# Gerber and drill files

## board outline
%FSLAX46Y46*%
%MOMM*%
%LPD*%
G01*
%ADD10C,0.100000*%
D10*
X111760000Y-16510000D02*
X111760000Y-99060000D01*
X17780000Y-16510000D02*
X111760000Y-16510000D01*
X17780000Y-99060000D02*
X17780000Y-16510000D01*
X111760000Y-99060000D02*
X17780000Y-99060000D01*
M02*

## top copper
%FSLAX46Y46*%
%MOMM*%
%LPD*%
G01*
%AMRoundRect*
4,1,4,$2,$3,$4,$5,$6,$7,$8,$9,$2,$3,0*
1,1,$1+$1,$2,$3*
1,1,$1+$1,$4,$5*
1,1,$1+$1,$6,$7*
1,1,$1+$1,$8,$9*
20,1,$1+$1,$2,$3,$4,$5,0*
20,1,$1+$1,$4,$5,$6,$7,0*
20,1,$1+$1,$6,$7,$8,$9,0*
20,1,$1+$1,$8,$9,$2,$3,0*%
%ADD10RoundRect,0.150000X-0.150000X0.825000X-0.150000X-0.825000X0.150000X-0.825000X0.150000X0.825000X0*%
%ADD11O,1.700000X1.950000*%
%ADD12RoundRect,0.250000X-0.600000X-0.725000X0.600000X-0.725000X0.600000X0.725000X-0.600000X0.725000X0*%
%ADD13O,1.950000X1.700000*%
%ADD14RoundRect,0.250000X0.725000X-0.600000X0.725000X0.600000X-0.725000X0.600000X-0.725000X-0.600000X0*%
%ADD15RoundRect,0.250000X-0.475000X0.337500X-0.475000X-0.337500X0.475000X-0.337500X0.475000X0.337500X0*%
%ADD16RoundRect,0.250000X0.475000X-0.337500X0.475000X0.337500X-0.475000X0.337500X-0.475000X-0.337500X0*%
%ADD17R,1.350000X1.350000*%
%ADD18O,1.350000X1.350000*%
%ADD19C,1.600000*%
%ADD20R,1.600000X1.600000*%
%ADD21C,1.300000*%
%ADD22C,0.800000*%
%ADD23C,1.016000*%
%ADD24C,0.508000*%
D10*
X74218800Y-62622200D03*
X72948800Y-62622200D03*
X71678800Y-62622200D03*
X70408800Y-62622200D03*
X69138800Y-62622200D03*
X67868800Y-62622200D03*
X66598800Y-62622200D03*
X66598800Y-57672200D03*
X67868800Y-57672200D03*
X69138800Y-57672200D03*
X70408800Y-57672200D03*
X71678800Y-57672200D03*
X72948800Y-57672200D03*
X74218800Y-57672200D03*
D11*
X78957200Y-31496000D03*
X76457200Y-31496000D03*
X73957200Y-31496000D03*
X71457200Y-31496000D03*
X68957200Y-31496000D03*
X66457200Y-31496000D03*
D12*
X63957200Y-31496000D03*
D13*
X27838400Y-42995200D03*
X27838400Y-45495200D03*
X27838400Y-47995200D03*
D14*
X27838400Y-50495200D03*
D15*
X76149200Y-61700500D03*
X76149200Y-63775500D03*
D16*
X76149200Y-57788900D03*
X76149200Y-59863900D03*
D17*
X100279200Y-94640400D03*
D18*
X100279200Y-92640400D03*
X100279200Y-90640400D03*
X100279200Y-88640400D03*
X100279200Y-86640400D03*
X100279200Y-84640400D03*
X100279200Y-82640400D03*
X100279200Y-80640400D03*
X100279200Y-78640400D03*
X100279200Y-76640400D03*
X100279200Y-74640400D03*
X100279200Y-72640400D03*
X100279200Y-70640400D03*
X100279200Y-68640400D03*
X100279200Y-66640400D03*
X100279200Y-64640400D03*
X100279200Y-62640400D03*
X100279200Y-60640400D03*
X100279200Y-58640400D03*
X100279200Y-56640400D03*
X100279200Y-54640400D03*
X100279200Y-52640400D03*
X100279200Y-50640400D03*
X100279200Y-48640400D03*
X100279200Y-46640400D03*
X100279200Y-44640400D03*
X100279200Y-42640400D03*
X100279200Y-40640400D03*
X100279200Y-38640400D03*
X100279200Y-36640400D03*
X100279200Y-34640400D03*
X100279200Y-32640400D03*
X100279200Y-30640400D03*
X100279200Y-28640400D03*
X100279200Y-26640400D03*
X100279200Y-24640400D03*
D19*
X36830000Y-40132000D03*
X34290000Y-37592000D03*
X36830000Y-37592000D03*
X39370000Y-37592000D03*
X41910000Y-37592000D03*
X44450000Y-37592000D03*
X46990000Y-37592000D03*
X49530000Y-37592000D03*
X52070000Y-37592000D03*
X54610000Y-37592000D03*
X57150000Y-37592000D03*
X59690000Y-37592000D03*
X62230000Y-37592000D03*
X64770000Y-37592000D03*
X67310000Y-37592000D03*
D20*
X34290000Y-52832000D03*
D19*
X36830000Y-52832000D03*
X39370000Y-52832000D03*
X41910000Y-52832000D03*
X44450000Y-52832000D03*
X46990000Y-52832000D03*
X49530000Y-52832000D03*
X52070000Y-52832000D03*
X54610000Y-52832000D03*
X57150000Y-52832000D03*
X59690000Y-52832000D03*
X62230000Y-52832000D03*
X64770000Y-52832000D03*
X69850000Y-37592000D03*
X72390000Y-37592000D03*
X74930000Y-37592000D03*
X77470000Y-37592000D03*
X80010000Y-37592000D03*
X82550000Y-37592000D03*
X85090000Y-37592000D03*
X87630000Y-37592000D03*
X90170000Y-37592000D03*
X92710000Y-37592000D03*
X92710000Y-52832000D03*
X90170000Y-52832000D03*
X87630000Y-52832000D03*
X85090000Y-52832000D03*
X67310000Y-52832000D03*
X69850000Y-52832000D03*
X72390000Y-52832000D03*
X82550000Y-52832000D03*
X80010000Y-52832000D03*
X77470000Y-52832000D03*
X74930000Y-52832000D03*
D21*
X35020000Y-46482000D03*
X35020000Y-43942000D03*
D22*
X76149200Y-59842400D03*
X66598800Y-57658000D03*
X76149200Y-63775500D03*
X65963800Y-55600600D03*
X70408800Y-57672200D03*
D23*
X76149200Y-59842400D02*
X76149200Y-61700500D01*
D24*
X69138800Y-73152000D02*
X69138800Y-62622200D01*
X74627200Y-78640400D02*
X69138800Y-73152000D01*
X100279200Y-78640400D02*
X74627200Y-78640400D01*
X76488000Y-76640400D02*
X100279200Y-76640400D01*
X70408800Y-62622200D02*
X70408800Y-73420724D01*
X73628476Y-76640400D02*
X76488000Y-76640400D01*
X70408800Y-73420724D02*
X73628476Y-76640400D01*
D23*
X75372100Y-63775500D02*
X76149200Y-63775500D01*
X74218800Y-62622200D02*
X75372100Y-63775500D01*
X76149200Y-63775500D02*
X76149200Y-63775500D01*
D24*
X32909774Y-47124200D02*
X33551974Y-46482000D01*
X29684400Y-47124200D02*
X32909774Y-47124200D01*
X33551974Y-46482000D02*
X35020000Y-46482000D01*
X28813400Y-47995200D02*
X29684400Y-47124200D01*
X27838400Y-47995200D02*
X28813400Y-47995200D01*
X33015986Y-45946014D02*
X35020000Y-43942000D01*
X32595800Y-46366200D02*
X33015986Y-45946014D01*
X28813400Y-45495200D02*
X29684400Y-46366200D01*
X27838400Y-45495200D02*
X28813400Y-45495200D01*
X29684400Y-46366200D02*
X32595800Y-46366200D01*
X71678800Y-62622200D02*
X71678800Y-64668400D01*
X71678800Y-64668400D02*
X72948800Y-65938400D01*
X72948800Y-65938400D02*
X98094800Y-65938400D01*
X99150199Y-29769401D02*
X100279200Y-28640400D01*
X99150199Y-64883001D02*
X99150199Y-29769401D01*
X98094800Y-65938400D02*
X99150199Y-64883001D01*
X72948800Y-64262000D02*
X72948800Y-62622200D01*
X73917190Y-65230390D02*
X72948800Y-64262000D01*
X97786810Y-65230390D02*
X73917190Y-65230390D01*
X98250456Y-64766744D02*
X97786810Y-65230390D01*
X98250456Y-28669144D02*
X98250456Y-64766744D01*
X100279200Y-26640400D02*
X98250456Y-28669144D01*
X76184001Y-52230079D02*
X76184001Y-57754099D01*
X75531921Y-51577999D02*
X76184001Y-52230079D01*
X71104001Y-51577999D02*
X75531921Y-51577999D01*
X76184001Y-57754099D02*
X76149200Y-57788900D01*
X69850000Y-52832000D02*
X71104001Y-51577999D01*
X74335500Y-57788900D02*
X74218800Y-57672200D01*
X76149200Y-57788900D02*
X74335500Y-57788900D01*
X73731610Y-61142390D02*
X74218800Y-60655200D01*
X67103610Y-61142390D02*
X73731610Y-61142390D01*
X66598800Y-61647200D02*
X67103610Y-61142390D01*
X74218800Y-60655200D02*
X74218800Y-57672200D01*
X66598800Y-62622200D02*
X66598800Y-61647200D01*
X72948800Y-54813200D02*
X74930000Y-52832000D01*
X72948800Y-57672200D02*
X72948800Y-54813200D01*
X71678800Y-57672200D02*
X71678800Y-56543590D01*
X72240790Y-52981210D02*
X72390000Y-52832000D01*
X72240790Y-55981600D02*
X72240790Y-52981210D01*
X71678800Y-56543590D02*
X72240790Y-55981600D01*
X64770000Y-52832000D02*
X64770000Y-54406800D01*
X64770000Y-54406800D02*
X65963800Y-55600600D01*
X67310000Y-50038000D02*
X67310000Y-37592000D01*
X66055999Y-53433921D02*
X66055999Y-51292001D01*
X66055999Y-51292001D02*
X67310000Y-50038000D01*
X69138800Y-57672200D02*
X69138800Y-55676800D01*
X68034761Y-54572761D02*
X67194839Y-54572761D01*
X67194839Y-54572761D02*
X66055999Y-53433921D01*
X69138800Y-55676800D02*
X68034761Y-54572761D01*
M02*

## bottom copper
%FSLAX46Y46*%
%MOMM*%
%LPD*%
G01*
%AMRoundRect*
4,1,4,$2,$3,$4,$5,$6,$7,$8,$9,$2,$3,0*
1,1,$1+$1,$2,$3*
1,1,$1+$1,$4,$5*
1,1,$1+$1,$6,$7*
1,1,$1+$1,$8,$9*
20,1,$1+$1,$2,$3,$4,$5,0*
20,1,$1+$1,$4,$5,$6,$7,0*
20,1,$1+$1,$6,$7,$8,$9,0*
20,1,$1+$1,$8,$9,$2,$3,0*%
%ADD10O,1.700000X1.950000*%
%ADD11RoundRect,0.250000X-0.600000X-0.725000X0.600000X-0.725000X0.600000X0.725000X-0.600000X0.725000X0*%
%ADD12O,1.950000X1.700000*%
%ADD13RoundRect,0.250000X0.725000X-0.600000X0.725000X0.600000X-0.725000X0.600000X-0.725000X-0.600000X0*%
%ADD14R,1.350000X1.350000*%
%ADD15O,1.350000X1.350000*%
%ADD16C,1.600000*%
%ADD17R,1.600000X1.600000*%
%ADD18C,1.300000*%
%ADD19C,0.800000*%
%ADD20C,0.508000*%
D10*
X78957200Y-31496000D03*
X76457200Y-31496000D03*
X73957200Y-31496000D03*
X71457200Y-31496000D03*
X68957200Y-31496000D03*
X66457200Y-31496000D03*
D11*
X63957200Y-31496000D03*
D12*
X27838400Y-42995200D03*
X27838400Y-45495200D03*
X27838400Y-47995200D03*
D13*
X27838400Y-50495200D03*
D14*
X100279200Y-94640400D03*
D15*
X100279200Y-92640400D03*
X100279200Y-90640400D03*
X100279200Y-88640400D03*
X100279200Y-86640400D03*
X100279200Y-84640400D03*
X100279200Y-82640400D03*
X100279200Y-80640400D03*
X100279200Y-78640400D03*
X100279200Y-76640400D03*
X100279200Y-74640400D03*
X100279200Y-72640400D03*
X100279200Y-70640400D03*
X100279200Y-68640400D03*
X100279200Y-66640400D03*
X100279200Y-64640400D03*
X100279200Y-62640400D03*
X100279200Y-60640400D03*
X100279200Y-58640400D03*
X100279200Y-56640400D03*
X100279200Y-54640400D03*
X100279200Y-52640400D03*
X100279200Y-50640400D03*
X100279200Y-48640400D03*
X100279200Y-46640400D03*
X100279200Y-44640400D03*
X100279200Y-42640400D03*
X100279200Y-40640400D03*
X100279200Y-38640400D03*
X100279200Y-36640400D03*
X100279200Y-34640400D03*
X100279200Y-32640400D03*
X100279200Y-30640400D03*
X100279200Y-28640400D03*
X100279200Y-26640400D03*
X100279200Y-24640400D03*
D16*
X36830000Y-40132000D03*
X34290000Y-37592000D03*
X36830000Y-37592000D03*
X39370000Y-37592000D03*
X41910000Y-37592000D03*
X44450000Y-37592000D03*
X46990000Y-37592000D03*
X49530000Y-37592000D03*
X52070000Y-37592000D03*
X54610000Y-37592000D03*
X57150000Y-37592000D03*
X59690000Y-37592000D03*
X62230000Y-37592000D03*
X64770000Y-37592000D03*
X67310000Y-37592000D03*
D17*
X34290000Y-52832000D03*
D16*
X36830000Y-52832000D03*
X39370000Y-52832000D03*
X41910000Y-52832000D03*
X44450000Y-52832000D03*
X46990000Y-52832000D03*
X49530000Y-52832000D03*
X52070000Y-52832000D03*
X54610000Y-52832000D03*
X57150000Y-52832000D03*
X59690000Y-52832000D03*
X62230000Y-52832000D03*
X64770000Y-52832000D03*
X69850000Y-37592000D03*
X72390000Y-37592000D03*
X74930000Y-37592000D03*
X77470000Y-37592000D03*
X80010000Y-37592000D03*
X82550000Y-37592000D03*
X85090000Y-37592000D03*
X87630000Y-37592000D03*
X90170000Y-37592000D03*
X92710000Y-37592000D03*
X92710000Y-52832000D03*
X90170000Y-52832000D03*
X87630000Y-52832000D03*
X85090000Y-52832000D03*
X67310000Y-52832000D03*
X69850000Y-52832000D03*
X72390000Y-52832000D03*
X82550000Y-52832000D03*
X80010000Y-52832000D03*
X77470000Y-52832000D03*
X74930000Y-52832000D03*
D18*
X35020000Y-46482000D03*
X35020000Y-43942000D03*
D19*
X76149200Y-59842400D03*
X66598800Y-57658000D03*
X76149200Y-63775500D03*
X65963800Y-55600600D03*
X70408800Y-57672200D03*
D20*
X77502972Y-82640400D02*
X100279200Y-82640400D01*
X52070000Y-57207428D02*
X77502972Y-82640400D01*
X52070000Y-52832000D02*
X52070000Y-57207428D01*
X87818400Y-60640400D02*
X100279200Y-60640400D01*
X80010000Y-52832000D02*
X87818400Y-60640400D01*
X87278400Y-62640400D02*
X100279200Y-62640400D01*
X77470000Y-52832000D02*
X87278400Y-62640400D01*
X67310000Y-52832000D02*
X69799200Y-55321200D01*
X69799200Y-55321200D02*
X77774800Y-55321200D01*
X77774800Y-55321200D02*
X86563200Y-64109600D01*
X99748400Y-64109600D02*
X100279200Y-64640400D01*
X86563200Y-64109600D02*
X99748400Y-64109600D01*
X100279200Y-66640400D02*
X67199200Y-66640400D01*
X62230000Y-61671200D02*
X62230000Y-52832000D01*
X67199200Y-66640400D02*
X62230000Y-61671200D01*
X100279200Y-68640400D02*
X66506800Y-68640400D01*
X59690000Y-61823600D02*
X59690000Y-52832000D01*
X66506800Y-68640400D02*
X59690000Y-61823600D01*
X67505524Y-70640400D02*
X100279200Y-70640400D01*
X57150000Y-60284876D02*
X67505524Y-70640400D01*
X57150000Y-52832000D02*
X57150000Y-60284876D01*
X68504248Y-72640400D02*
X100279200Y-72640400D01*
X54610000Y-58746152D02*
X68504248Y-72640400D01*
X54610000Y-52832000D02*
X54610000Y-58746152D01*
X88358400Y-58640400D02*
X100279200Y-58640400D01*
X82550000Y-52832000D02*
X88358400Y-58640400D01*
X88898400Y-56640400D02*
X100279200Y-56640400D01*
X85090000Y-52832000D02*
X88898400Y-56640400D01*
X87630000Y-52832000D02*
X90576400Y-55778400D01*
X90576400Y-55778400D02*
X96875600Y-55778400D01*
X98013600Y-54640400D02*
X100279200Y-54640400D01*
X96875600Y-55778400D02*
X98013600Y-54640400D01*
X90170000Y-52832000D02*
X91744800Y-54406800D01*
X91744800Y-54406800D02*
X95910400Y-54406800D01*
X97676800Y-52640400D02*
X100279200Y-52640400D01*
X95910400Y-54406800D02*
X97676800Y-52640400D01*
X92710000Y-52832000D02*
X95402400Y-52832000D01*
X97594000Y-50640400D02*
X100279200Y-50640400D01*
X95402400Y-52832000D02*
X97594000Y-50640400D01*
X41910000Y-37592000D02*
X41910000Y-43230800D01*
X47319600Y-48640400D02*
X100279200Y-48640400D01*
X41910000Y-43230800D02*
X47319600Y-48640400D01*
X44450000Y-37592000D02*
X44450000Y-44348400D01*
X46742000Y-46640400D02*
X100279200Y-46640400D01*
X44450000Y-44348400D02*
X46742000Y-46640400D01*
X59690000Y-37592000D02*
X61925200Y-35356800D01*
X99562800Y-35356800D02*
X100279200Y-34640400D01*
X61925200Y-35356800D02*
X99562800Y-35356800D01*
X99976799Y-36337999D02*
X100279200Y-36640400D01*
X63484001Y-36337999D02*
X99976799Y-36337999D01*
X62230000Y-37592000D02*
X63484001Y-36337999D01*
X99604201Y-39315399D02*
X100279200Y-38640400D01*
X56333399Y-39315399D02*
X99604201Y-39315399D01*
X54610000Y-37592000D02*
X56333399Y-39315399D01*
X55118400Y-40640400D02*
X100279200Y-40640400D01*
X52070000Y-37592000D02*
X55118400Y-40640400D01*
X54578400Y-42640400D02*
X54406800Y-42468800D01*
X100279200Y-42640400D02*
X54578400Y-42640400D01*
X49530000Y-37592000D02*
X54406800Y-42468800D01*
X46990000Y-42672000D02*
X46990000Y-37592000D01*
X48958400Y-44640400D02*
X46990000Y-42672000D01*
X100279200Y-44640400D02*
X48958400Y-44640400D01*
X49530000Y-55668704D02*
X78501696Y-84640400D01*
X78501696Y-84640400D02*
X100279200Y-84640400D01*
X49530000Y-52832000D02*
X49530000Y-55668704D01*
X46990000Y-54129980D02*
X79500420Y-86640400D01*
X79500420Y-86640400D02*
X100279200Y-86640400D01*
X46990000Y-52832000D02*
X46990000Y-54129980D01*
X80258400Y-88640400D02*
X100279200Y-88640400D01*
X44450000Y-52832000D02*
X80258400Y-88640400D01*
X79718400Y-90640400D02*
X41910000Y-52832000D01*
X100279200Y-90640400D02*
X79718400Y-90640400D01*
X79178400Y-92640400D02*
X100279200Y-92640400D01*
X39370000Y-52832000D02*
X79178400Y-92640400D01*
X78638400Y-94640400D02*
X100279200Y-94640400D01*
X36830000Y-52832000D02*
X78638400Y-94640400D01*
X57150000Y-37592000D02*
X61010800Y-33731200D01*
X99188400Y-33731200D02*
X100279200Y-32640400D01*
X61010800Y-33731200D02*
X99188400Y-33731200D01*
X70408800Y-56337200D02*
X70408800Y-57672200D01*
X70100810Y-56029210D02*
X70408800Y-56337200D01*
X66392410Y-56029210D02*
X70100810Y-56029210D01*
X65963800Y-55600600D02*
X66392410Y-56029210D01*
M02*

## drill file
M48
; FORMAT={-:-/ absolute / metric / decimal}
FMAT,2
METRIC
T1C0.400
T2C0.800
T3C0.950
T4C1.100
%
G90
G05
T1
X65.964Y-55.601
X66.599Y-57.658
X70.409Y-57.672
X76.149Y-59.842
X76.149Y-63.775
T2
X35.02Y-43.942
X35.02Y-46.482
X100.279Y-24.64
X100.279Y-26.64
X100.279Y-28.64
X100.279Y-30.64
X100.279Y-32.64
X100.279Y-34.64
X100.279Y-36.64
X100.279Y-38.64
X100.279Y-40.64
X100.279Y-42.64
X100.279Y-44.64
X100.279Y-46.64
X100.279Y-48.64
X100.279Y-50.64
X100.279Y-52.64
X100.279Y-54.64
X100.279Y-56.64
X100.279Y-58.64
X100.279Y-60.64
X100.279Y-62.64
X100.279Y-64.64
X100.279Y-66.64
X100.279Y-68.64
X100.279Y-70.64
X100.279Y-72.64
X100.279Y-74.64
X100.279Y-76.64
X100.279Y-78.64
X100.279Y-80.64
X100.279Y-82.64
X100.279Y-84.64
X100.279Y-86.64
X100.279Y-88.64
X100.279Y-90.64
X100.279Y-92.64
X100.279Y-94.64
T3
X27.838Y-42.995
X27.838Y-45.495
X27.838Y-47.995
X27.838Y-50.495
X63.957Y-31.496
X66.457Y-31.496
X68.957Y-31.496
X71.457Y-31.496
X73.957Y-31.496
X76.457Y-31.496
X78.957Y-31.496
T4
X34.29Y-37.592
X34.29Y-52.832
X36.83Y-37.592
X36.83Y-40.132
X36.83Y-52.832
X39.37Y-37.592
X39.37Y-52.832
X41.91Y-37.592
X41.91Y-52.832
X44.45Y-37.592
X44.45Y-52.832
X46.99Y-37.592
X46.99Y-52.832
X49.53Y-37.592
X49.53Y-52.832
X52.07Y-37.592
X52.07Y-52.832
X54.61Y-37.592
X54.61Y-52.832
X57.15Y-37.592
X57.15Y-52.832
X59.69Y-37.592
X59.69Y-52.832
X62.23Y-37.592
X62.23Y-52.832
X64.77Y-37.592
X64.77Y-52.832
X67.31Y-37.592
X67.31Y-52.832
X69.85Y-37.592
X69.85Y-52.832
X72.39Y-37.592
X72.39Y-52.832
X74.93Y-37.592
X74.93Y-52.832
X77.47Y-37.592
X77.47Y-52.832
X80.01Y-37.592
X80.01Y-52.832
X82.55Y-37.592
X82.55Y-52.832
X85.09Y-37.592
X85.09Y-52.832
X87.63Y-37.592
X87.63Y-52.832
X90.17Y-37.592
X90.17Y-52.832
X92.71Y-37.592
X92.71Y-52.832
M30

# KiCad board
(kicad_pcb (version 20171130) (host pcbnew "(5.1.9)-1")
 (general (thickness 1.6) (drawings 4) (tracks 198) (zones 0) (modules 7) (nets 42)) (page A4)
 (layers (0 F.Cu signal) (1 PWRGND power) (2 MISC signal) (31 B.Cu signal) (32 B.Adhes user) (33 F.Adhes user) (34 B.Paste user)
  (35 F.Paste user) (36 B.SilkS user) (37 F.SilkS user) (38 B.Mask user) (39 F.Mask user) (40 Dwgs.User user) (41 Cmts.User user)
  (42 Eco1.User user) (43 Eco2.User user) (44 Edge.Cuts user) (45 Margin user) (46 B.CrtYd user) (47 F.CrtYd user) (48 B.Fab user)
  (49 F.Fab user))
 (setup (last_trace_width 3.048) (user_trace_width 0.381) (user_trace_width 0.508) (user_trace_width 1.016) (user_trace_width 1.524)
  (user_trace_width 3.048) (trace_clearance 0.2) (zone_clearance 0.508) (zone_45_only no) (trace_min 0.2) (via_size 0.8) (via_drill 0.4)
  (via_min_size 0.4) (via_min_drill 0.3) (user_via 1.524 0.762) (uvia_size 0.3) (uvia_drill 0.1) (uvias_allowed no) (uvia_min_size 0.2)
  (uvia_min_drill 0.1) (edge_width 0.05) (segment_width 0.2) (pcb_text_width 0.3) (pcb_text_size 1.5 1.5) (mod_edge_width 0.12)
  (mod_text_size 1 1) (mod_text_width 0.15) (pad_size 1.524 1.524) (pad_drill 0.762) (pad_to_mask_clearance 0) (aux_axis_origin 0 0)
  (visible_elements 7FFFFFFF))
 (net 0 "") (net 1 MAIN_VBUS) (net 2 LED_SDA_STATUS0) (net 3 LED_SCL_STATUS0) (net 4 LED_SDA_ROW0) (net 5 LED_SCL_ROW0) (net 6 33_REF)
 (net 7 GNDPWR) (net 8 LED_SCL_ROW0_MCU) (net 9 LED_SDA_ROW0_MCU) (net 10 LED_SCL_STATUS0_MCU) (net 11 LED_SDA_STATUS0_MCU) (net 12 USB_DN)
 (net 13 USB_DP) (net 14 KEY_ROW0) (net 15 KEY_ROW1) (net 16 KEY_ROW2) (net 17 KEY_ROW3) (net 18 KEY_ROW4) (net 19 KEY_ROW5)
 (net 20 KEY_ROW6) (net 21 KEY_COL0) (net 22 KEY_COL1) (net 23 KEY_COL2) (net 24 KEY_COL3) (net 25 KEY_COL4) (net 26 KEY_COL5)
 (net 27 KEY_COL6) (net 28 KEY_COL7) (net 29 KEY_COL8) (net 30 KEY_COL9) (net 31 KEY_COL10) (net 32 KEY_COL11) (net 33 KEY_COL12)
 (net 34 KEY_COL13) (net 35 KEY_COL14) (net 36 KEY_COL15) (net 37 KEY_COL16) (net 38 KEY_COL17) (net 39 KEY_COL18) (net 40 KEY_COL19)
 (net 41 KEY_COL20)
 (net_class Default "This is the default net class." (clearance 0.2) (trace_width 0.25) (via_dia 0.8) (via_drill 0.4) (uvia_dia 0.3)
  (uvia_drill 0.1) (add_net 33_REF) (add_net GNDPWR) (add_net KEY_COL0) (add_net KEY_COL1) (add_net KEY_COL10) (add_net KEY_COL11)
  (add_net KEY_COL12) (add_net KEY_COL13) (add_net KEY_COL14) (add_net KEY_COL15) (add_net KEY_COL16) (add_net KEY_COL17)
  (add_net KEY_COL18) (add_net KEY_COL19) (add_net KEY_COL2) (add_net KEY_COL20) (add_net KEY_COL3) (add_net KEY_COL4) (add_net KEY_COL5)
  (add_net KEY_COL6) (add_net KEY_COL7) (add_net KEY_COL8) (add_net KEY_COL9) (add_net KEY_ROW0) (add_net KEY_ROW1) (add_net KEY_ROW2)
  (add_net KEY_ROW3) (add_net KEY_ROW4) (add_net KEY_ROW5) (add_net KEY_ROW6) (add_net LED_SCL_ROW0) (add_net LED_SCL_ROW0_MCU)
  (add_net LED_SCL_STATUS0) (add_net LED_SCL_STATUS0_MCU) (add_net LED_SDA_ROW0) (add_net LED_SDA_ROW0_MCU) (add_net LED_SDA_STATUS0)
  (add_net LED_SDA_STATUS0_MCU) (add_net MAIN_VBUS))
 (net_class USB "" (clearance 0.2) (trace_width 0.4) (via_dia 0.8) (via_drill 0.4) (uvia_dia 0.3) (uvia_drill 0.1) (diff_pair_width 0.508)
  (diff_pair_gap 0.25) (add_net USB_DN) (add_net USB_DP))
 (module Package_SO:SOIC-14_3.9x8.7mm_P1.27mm (layer F.Cu) (at 70.4088 60.1472 270)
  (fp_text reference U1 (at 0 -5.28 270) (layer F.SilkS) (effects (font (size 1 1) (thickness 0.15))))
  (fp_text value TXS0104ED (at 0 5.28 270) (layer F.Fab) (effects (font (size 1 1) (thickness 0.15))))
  (pad 14 smd roundrect (at 2.475 -3.81 270) (size 1.95 0.6) (layers F.Cu F.Paste F.Mask) (roundrect_rratio 0.25) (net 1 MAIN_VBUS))
  (pad 13 smd roundrect (at 2.475 -2.54 270) (size 1.95 0.6) (layers F.Cu F.Paste F.Mask) (roundrect_rratio 0.25) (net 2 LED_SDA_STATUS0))
  (pad 12 smd roundrect (at 2.475 -1.27 270) (size 1.95 0.6) (layers F.Cu F.Paste F.Mask) (roundrect_rratio 0.25) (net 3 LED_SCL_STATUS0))
  (pad 11 smd roundrect (at 2.475 0 270) (size 1.95 0.6) (layers F.Cu F.Paste F.Mask) (roundrect_rratio 0.25) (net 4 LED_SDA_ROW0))
  (pad 10 smd roundrect (at 2.475 1.27 270) (size 1.95 0.6) (layers F.Cu F.Paste F.Mask) (roundrect_rratio 0.25) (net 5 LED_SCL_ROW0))
  (pad 9 smd roundrect (at 2.475 2.54 270) (size 1.95 0.6) (layers F.Cu F.Paste F.Mask) (roundrect_rratio 0.25))
  (pad 8 smd roundrect (at 2.475 3.81 270) (size 1.95 0.6) (layers F.Cu F.Paste F.Mask) (roundrect_rratio 0.25) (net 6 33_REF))
  (pad 7 smd roundrect (at -2.475 3.81 270) (size 1.95 0.6) (layers F.Cu F.Paste F.Mask) (roundrect_rratio 0.25) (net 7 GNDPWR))
  (pad 6 smd roundrect (at -2.475 2.54 270) (size 1.95 0.6) (layers F.Cu F.Paste F.Mask) (roundrect_rratio 0.25))
  (pad 5 smd roundrect (at -2.475 1.27 270) (size 1.95 0.6) (layers F.Cu F.Paste F.Mask) (roundrect_rratio 0.25) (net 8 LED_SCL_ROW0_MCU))
  (pad 4 smd roundrect (at -2.475 0 270) (size 1.95 0.6) (layers F.Cu F.Paste F.Mask) (roundrect_rratio 0.25) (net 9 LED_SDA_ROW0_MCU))
  (pad 3 smd roundrect (at -2.475 -1.27 270) (size 1.95 0.6) (layers F.Cu F.Paste F.Mask) (roundrect_rratio 0.25)
   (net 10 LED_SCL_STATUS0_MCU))
  (pad 2 smd roundrect (at -2.475 -2.54 270) (size 1.95 0.6) (layers F.Cu F.Paste F.Mask) (roundrect_rratio 0.25)
   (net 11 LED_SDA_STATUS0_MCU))
  (pad 1 smd roundrect (at -2.475 -3.81 270) (size 1.95 0.6) (layers F.Cu F.Paste F.Mask) (roundrect_rratio 0.25) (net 6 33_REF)))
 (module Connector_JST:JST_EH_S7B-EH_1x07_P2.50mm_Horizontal (layer F.Cu) (at 63.9572 31.496)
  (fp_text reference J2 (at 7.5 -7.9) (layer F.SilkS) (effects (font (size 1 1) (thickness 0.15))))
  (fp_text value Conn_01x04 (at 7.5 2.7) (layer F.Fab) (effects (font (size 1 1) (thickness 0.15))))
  (pad 7 thru_hole oval (at 15 0) (size 1.7 1.95) (drill 0.95) (layers *.Cu *.Mask))
  (pad 6 thru_hole oval (at 12.5 0) (size 1.7 1.95) (drill 0.95) (layers *.Cu *.Mask))
  (pad 5 thru_hole oval (at 10 0) (size 1.7 1.95) (drill 0.95) (layers *.Cu *.Mask))
  (pad 4 thru_hole oval (at 7.5 0) (size 1.7 1.95) (drill 0.95) (layers *.Cu *.Mask))
  (pad 3 thru_hole oval (at 5 0) (size 1.7 1.95) (drill 0.95) (layers *.Cu *.Mask))
  (pad 2 thru_hole oval (at 2.5 0) (size 1.7 1.95) (drill 0.95) (layers *.Cu *.Mask))
  (pad 1 thru_hole roundrect (at 0 0) (size 1.7 1.95) (drill 0.95) (layers *.Cu *.Mask) (roundrect_rratio 0.1470588235294118)))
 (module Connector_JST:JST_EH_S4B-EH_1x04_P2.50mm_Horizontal (layer F.Cu) (at 27.8384 50.4952 90)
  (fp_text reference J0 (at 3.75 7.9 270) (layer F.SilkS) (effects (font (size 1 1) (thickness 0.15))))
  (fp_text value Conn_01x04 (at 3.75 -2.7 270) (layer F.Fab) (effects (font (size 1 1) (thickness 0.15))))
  (pad 4 thru_hole oval (at 7.5 0 90) (size 1.7 1.95) (drill 0.95) (layers *.Cu *.Mask) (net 7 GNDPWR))
  (pad 3 thru_hole oval (at 5 0 90) (size 1.7 1.95) (drill 0.95) (layers *.Cu *.Mask) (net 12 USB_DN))
  (pad 2 thru_hole oval (at 2.5 0 90) (size 1.7 1.95) (drill 0.95) (layers *.Cu *.Mask) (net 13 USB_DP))
  (pad 1 thru_hole roundrect (at 0 0 90) (size 1.7 1.95) (drill 0.95) (layers *.Cu *.Mask) (roundrect_rratio 0.1470588235294118)
   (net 1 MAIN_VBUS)))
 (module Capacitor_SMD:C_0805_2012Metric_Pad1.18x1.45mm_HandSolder (layer F.Cu) (at 76.1492 62.738 270)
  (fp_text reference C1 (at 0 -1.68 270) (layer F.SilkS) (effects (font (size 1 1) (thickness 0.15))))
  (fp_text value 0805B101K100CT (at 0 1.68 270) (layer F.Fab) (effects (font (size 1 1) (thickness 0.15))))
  (pad 1 smd roundrect (at -1.0375 0 270) (size 1.175 1.45) (layers F.Cu F.Paste F.Mask) (roundrect_rratio 0.2127659574468085)
   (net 7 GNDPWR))
  (pad 2 smd roundrect (at 1.0375 0 270) (size 1.175 1.45) (layers F.Cu F.Paste F.Mask) (roundrect_rratio 0.2127659574468085)
   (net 1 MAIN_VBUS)))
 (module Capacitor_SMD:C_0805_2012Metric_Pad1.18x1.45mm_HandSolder (layer F.Cu) (at 76.1492 58.8264 90)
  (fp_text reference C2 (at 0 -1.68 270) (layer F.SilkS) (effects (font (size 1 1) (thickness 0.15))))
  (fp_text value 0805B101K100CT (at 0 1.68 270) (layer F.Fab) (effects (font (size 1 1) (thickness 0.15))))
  (pad 2 smd roundrect (at 1.0375 0 90) (size 1.175 1.45) (layers F.Cu F.Paste F.Mask) (roundrect_rratio 0.2127659574468085) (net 6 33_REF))
  (pad 1 smd roundrect (at -1.0375 0 90) (size 1.175 1.45) (layers F.Cu F.Paste F.Mask) (roundrect_rratio 0.2127659574468085) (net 7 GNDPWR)))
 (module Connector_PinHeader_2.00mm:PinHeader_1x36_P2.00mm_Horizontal (layer B.Cu) (at 100.2792 94.6404)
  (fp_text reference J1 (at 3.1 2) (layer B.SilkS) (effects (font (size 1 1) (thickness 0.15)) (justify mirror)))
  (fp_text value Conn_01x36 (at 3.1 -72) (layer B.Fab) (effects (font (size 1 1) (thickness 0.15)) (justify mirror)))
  (pad 1 thru_hole rect (at 0 0) (size 1.35 1.35) (drill 0.8) (layers *.Cu *.Mask) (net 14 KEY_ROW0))
  (pad 2 thru_hole oval (at 0 -2) (size 1.35 1.35) (drill 0.8) (layers *.Cu *.Mask) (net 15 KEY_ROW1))
  (pad 3 thru_hole oval (at 0 -4) (size 1.35 1.35) (drill 0.8) (layers *.Cu *.Mask) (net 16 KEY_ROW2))
  (pad 4 thru_hole oval (at 0 -6) (size 1.35 1.35) (drill 0.8) (layers *.Cu *.Mask) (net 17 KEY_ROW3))
  (pad 5 thru_hole oval (at 0 -8) (size 1.35 1.35) (drill 0.8) (layers *.Cu *.Mask) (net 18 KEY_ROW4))
  (pad 6 thru_hole oval (at 0 -10) (size 1.35 1.35) (drill 0.8) (layers *.Cu *.Mask) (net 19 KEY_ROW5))
  (pad 7 thru_hole oval (at 0 -12) (size 1.35 1.35) (drill 0.8) (layers *.Cu *.Mask) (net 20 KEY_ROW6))
  (pad 8 thru_hole oval (at 0 -14) (size 1.35 1.35) (drill 0.8) (layers *.Cu *.Mask) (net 1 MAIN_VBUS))
  (pad 9 thru_hole oval (at 0 -16) (size 1.35 1.35) (drill 0.8) (layers *.Cu *.Mask) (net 5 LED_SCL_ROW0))
  (pad 10 thru_hole oval (at 0 -18) (size 1.35 1.35) (drill 0.8) (layers *.Cu *.Mask) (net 4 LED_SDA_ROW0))
  (pad 11 thru_hole oval (at 0 -20) (size 1.35 1.35) (drill 0.8) (layers *.Cu *.Mask) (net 7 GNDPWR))
  (pad 12 thru_hole oval (at 0 -22) (size 1.35 1.35) (drill 0.8) (layers *.Cu *.Mask) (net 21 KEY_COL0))
  (pad 13 thru_hole oval (at 0 -24) (size 1.35 1.35) (drill 0.8) (layers *.Cu *.Mask) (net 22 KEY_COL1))
  (pad 14 thru_hole oval (at 0 -26) (size 1.35 1.35) (drill 0.8) (layers *.Cu *.Mask) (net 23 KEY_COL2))
  (pad 15 thru_hole oval (at 0 -28) (size 1.35 1.35) (drill 0.8) (layers *.Cu *.Mask) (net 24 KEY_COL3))
  (pad 16 thru_hole oval (at 0 -30) (size 1.35 1.35) (drill 0.8) (layers *.Cu *.Mask) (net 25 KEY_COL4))
  (pad 17 thru_hole oval (at 0 -32) (size 1.35 1.35) (drill 0.8) (layers *.Cu *.Mask) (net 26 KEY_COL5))
  (pad 18 thru_hole oval (at 0 -34) (size 1.35 1.35) (drill 0.8) (layers *.Cu *.Mask) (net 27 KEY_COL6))
  (pad 19 thru_hole oval (at 0 -36) (size 1.35 1.35) (drill 0.8) (layers *.Cu *.Mask) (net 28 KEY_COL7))
  (pad 20 thru_hole oval (at 0 -38) (size 1.35 1.35) (drill 0.8) (layers *.Cu *.Mask) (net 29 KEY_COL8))
  (pad 21 thru_hole oval (at 0 -40) (size 1.35 1.35) (drill 0.8) (layers *.Cu *.Mask) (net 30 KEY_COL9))
  (pad 22 thru_hole oval (at 0 -42) (size 1.35 1.35) (drill 0.8) (layers *.Cu *.Mask) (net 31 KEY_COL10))
  (pad 23 thru_hole oval (at 0 -44) (size 1.35 1.35) (drill 0.8) (layers *.Cu *.Mask) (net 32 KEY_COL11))
  (pad 24 thru_hole oval (at 0 -46) (size 1.35 1.35) (drill 0.8) (layers *.Cu *.Mask) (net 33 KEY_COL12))
  (pad 25 thru_hole oval (at 0 -48) (size 1.35 1.35) (drill 0.8) (layers *.Cu *.Mask) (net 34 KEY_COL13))
  (pad 26 thru_hole oval (at 0 -50) (size 1.35 1.35) (drill 0.8) (layers *.Cu *.Mask) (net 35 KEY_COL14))
  (pad 27 thru_hole oval (at 0 -52) (size 1.35 1.35) (drill 0.8) (layers *.Cu *.Mask) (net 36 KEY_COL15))
  (pad 28 thru_hole oval (at 0 -54) (size 1.35 1.35) (drill 0.8) (layers *.Cu *.Mask) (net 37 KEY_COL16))
  (pad 29 thru_hole oval (at 0 -56) (size 1.35 1.35) (drill 0.8) (layers *.Cu *.Mask) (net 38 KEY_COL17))
  (pad 30 thru_hole oval (at 0 -58) (size 1.35 1.35) (drill 0.8) (layers *.Cu *.Mask) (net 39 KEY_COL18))
  (pad 31 thru_hole oval (at 0 -60) (size 1.35 1.35) (drill 0.8) (layers *.Cu *.Mask) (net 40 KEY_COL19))
  (pad 32 thru_hole oval (at 0 -62) (size 1.35 1.35) (drill 0.8) (layers *.Cu *.Mask) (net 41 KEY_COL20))
  (pad 33 thru_hole oval (at 0 -64) (size 1.35 1.35) (drill 0.8) (layers *.Cu *.Mask) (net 1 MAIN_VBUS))
  (pad 34 thru_hole oval (at 0 -66) (size 1.35 1.35) (drill 0.8) (layers *.Cu *.Mask) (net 3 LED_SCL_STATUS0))
  (pad 35 thru_hole oval (at 0 -68) (size 1.35 1.35) (drill 0.8) (layers *.Cu *.Mask) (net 2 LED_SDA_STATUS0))
  (pad 36 thru_hole oval (at 0 -70) (size 1.35 1.35) (drill 0.8) (layers *.Cu *.Mask) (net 7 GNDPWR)))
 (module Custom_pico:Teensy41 (layer F.Cu) (at 63.5 45.212)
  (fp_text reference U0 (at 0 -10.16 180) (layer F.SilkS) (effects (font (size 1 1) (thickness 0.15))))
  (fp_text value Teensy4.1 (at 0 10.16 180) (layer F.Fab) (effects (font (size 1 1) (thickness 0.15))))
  (pad 49 thru_hole circle (at -26.67 -5.08) (size 1.6 1.6) (drill 1.1) (layers *.Cu *.Mask) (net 1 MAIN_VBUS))
  (pad 48 thru_hole circle (at -29.21 -7.62) (size 1.6 1.6) (drill 1.1) (layers *.Cu *.Mask))
  (pad 47 thru_hole circle (at -26.67 -7.62) (size 1.6 1.6) (drill 1.1) (layers *.Cu *.Mask) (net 7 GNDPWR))
  (pad 46 thru_hole circle (at -24.13 -7.62) (size 1.6 1.6) (drill 1.1) (layers *.Cu *.Mask))
  (pad 45 thru_hole circle (at -21.59 -7.62) (size 1.6 1.6) (drill 1.1) (layers *.Cu *.Mask) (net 33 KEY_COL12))
  (pad 44 thru_hole circle (at -19.05 -7.62) (size 1.6 1.6) (drill 1.1) (layers *.Cu *.Mask) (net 34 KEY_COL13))
  (pad 43 thru_hole circle (at -16.51 -7.62) (size 1.6 1.6) (drill 1.1) (layers *.Cu *.Mask) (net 35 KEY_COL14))
  (pad 42 thru_hole circle (at -13.97 -7.62) (size 1.6 1.6) (drill 1.1) (layers *.Cu *.Mask) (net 36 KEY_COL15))
  (pad 41 thru_hole circle (at -11.43 -7.62) (size 1.6 1.6) (drill 1.1) (layers *.Cu *.Mask) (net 37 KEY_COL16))
  (pad 40 thru_hole circle (at -8.89 -7.62) (size 1.6 1.6) (drill 1.1) (layers *.Cu *.Mask) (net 38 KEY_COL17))
  (pad 39 thru_hole circle (at -6.35 -7.62) (size 1.6 1.6) (drill 1.1) (layers *.Cu *.Mask) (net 41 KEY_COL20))
  (pad 38 thru_hole circle (at -3.81 -7.62) (size 1.6 1.6) (drill 1.1) (layers *.Cu *.Mask) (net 40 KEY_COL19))
  (pad 37 thru_hole circle (at -1.27 -7.62) (size 1.6 1.6) (drill 1.1) (layers *.Cu *.Mask) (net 39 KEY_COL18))
  (pad 36 thru_hole circle (at 1.27 -7.62) (size 1.6 1.6) (drill 1.1) (layers *.Cu *.Mask))
  (pad 35 thru_hole circle (at 3.81 -7.62) (size 1.6 1.6) (drill 1.1) (layers *.Cu *.Mask) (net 8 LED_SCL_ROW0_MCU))
  (pad 1 thru_hole rect (at -29.21 7.62) (size 1.6 1.6) (drill 1.1) (layers *.Cu *.Mask))
  (pad 2 thru_hole circle (at -26.67 7.62) (size 1.6 1.6) (drill 1.1) (layers *.Cu *.Mask) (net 14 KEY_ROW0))
  (pad 3 thru_hole circle (at -24.13 7.62) (size 1.6 1.6) (drill 1.1) (layers *.Cu *.Mask) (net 15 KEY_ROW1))
  (pad 4 thru_hole circle (at -21.59 7.62) (size 1.6 1.6) (drill 1.1) (layers *.Cu *.Mask) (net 16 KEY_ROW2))
  (pad 5 thru_hole circle (at -19.05 7.62) (size 1.6 1.6) (drill 1.1) (layers *.Cu *.Mask) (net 17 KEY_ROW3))
  (pad 6 thru_hole circle (at -16.51 7.62) (size 1.6 1.6) (drill 1.1) (layers *.Cu *.Mask) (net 18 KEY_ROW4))
  (pad 7 thru_hole circle (at -13.97 7.62) (size 1.6 1.6) (drill 1.1) (layers *.Cu *.Mask) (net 19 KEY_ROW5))
  (pad 8 thru_hole circle (at -11.43 7.62) (size 1.6 1.6) (drill 1.1) (layers *.Cu *.Mask) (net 20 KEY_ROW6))
  (pad 9 thru_hole circle (at -8.89 7.62) (size 1.6 1.6) (drill 1.1) (layers *.Cu *.Mask) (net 21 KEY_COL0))
  (pad 10 thru_hole circle (at -6.35 7.62) (size 1.6 1.6) (drill 1.1) (layers *.Cu *.Mask) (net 22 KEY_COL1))
  (pad 11 thru_hole circle (at -3.81 7.62) (size 1.6 1.6) (drill 1.1) (layers *.Cu *.Mask) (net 23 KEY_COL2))
  (pad 12 thru_hole circle (at -1.27 7.62) (size 1.6 1.6) (drill 1.1) (layers *.Cu *.Mask) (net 24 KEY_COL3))
  (pad 13 thru_hole circle (at 1.27 7.62) (size 1.6 1.6) (drill 1.1) (layers *.Cu *.Mask) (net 9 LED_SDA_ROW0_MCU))
  (pad 34 thru_hole circle (at 6.35 -7.62) (size 1.6 1.6) (drill 1.1) (layers *.Cu *.Mask))
  (pad 33 thru_hole circle (at 8.89 -7.62) (size 1.6 1.6) (drill 1.1) (layers *.Cu *.Mask))
  (pad 32 thru_hole circle (at 11.43 -7.62) (size 1.6 1.6) (drill 1.1) (layers *.Cu *.Mask))
  (pad 31 thru_hole circle (at 13.97 -7.62) (size 1.6 1.6) (drill 1.1) (layers *.Cu *.Mask))
  (pad 30 thru_hole circle (at 16.51 -7.62) (size 1.6 1.6) (drill 1.1) (layers *.Cu *.Mask))
  (pad 29 thru_hole circle (at 19.05 -7.62) (size 1.6 1.6) (drill 1.1) (layers *.Cu *.Mask))
  (pad 28 thru_hole circle (at 21.59 -7.62) (size 1.6 1.6) (drill 1.1) (layers *.Cu *.Mask))
  (pad 27 thru_hole circle (at 24.13 -7.62) (size 1.6 1.6) (drill 1.1) (layers *.Cu *.Mask))
  (pad 26 thru_hole circle (at 26.67 -7.62) (size 1.6 1.6) (drill 1.1) (layers *.Cu *.Mask))
  (pad 25 thru_hole circle (at 29.21 -7.62) (size 1.6 1.6) (drill 1.1) (layers *.Cu *.Mask))
  (pad 24 thru_hole circle (at 29.21 7.62) (size 1.6 1.6) (drill 1.1) (layers *.Cu *.Mask) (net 32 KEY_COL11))
  (pad 23 thru_hole circle (at 26.67 7.62) (size 1.6 1.6) (drill 1.1) (layers *.Cu *.Mask) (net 31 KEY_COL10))
  (pad 22 thru_hole circle (at 24.13 7.62) (size 1.6 1.6) (drill 1.1) (layers *.Cu *.Mask) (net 30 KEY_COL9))
  (pad 21 thru_hole circle (at 21.59 7.62) (size 1.6 1.6) (drill 1.1) (layers *.Cu *.Mask) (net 29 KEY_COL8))
  (pad 14 thru_hole circle (at 3.81 7.62) (size 1.6 1.6) (drill 1.1) (layers *.Cu *.Mask) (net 25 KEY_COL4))
  (pad 15 thru_hole circle (at 6.35 7.62) (size 1.6 1.6) (drill 1.1) (layers *.Cu *.Mask) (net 6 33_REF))
  (pad 16 thru_hole circle (at 8.89 7.62) (size 1.6 1.6) (drill 1.1) (layers *.Cu *.Mask) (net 10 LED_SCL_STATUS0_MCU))
  (pad 20 thru_hole circle (at 19.05 7.62) (size 1.6 1.6) (drill 1.1) (layers *.Cu *.Mask) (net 28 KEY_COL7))
  (pad 19 thru_hole circle (at 16.51 7.62) (size 1.6 1.6) (drill 1.1) (layers *.Cu *.Mask) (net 27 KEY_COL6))
  (pad 18 thru_hole circle (at 13.97 7.62) (size 1.6 1.6) (drill 1.1) (layers *.Cu *.Mask) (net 26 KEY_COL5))
  (pad 17 thru_hole circle (at 11.43 7.62) (size 1.6 1.6) (drill 1.1) (layers *.Cu *.Mask) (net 11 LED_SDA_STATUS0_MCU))
  (pad 67 thru_hole circle (at -28.48 1.27) (size 1.3 1.3) (drill 0.8) (layers *.Cu *.Mask) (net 13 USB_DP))
  (pad 66 thru_hole circle (at -28.48 -1.27) (size 1.3 1.3) (drill 0.8) (layers *.Cu *.Mask) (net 12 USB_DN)))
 (gr_line (start 111.76 16.51) (end 111.76 99.06) (layer Edge.Cuts) (width 0.1))
 (gr_line (start 17.78 16.51) (end 111.76 16.51) (layer Edge.Cuts) (width 0.1))
 (gr_line (start 17.78 99.06) (end 17.78 16.51) (layer Edge.Cuts) (width 0.1))
 (gr_line (start 111.76 99.06) (end 17.78 99.06) (layer Edge.Cuts) (width 0.1))
 (via (at 76.1492 59.8424) (size 0.8) (drill 0.4) (layers F.Cu B.Cu) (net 7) (status 30))
 (via (at 66.5988 57.658) (size 0.8) (drill 0.4) (layers F.Cu B.Cu) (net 7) (status 30))
 (segment (start 77.502972 82.6404) (end 100.2792 82.6404) (width 0.508) (layer B.Cu) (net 20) (status 20))
 (segment (start 52.07 57.207428) (end 77.502972 82.6404) (width 0.508) (layer B.Cu) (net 20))
 (segment (start 52.07 52.832) (end 52.07 57.207428) (width 0.508) (layer B.Cu) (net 20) (status 10))
 (segment (start 27.8384 37.6428) (end 27.8384 42.9952) (width 1.524) (layer MISC) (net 7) (status 20))
 (segment (start 29.651201 35.829999) (end 27.8384 37.6428) (width 1.524) (layer MISC) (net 7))
 (segment (start 36.185599 35.829999) (end 29.651201 35.829999) (width 1.524) (layer MISC) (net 7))
 (segment (start 36.83 36.4744) (end 36.185599 35.829999) (width 1.524) (layer MISC) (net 7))
 (segment (start 36.83 37.592) (end 36.83 36.4744) (width 1.524) (layer MISC) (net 7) (status 10))
 (segment (start 102.362 21.59) (end 105.156 24.384) (width 3.048) (layer MISC) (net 7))
 (segment (start 105.156 24.384) (end 105.156 74.7268) (width 3.048) (layer MISC) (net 7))
 (segment (start 100.2792 74.6404) (end 101.4628 74.6404) (width 1.524) (layer MISC) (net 7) (status 10))
 (segment (start 101.916122 74.7268) (end 101.829722 74.6404) (width 3.048) (layer MISC) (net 7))
 (segment (start 105.156 74.7268) (end 101.916122 74.7268) (width 3.048) (layer MISC) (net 7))
 (segment (start 100.2792 24.6404) (end 100.2792 21.844) (width 1.524) (layer MISC) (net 7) (status 10))
 (segment (start 100.2792 21.844) (end 100.5332 21.59) (width 1.524) (layer MISC) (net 7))
 (segment (start 100.5332 21.59) (end 102.362 21.59) (width 3.048) (layer MISC) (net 7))
 (segment (start 66.5988 57.658) (end 66.5988 58.8772) (width 1.016) (layer MISC) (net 7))
 (segment (start 67.564 59.8424) (end 76.1492 59.8424) (width 1.016) (layer MISC) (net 7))
 (segment (start 66.5988 58.8772) (end 67.564 59.8424) (width 1.016) (layer MISC) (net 7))
 (segment (start 76.1492 59.8424) (end 76.1492 61.7005) (width 1.016) (layer F.Cu) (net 7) (status 30))
 (segment (start 100.2792 74.6404) (end 89.3724 74.6404) (width 1.016) (layer MISC) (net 7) (status 10))
 (segment (start 76.1492 59.8424) (end 79.1972 59.8424) (width 1.016) (layer MISC) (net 7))
 (segment (start 79.1972 59.8424) (end 82.3976 63.0428) (width 1.016) (layer MISC) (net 7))
 (segment (start 82.3976 63.0428) (end 82.3976 73.6092) (width 1.016) (layer MISC) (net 7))
 (segment (start 83.4288 74.6404) (end 89.3724 74.6404) (width 1.016) (layer MISC) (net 7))
 (segment (start 82.3976 73.6092) (end 83.4288 74.6404) (width 1.016) (layer MISC) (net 7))
 (segment (start 54.61 21.59) (end 100.5332 21.59) (width 3.048) (layer MISC) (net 7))
 (segment (start 51.636478 21.59) (end 54.61 21.59) (width 3.048) (layer MISC) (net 7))
 (segment (start 36.83 36.396478) (end 51.636478 21.59) (width 3.048) (layer MISC) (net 7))
 (segment (start 36.83 36.4744) (end 36.83 36.396478) (width 3.048) (layer MISC) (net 7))
 (segment (start 87.8184 60.6404) (end 100.2792 60.6404) (width 0.508) (layer B.Cu) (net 27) (status 20))
 (segment (start 80.01 52.832) (end 87.8184 60.6404) (width 0.508) (layer B.Cu) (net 27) (status 10))
 (segment (start 87.2784 62.6404) (end 100.2792 62.6404) (width 0.508) (layer B.Cu) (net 26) (status 20))
 (segment (start 77.47 52.832) (end 87.2784 62.6404) (width 0.508) (layer B.Cu) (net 26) (status 10))
 (segment (start 67.31 52.832) (end 69.7992 55.3212) (width 0.508) (layer B.Cu) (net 25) (status 10))
 (segment (start 69.7992 55.3212) (end 77.7748 55.3212) (width 0.508) (layer B.Cu) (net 25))
 (segment (start 77.7748 55.3212) (end 86.5632 64.1096) (width 0.508) (layer B.Cu) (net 25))
 (segment (start 99.7484 64.1096) (end 100.2792 64.6404) (width 0.508) (layer B.Cu) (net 25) (status 20))
 (segment (start 86.5632 64.1096) (end 99.7484 64.1096) (width 0.508) (layer B.Cu) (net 25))
 (segment (start 100.2792 66.6404) (end 67.1992 66.6404) (width 0.508) (layer B.Cu) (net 24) (status 10))
 (segment (start 62.23 61.6712) (end 62.23 52.832) (width 0.508) (layer B.Cu) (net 24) (status 20))
 (segment (start 67.1992 66.6404) (end 62.23 61.6712) (width 0.508) (layer B.Cu) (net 24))
 (segment (start 100.2792 68.6404) (end 66.5068 68.6404) (width 0.508) (layer B.Cu) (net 23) (status 10))
 (segment (start 59.69 61.8236) (end 59.69 52.832) (width 0.508) (layer B.Cu) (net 23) (status 20))
 (segment (start 66.5068 68.6404) (end 59.69 61.8236) (width 0.508) (layer B.Cu) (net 23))
 (segment (start 67.505524 70.6404) (end 100.2792 70.6404) (width 0.508) (layer B.Cu) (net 22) (status 20))
 (segment (start 57.15 60.284876) (end 67.505524 70.6404) (width 0.508) (layer B.Cu) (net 22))
 (segment (start 57.15 52.832) (end 57.15 60.284876) (width 0.508) (layer B.Cu) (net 22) (status 10))
 (segment (start 68.504248 72.6404) (end 100.2792 72.6404) (width 0.508) (layer B.Cu) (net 21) (status 20))
 (segment (start 54.61 58.746152) (end 68.504248 72.6404) (width 0.508) (layer B.Cu) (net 21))
 (segment (start 54.61 52.832) (end 54.61 58.746152) (width 0.508) (layer B.Cu) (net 21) (status 10))
 (segment (start 88.3584 58.6404) (end 100.2792 58.6404) (width 0.508) (layer B.Cu) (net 28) (status 20))
 (segment (start 82.55 52.832) (end 88.3584 58.6404) (width 0.508) (layer B.Cu) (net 28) (status 10))
 (segment (start 88.8984 56.6404) (end 100.2792 56.6404) (width 0.508) (layer B.Cu) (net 29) (status 20))
 (segment (start 85.09 52.832) (end 88.8984 56.6404) (width 0.508) (layer B.Cu) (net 29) (status 10))
 (segment (start 87.63 52.832) (end 90.5764 55.7784) (width 0.508) (layer B.Cu) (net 30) (status 10))
 (segment (start 90.5764 55.7784) (end 96.8756 55.7784) (width 0.508) (layer B.Cu) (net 30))
 (segment (start 98.0136 54.6404) (end 100.2792 54.6404) (width 0.508) (layer B.Cu) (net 30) (status 20))
 (segment (start 96.8756 55.7784) (end 98.0136 54.6404) (width 0.508) (layer B.Cu) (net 30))
 (segment (start 90.17 52.832) (end 91.7448 54.4068) (width 0.508) (layer B.Cu) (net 31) (status 10))
 (segment (start 91.7448 54.4068) (end 95.9104 54.4068) (width 0.508) (layer B.Cu) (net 31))
 (segment (start 97.6768 52.6404) (end 100.2792 52.6404) (width 0.508) (layer B.Cu) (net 31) (status 20))
 (segment (start 95.9104 54.4068) (end 97.6768 52.6404) (width 0.508) (layer B.Cu) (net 31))
 (segment (start 92.71 52.832) (end 95.4024 52.832) (width 0.508) (layer B.Cu) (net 32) (status 10))
 (segment (start 97.594 50.6404) (end 100.2792 50.6404) (width 0.508) (layer B.Cu) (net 32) (status 20))
 (segment (start 95.4024 52.832) (end 97.594 50.6404) (width 0.508) (layer B.Cu) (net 32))
 (segment (start 41.91 37.592) (end 41.91 43.2308) (width 0.508) (layer B.Cu) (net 33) (status 10))
 (segment (start 47.3196 48.6404) (end 100.2792 48.6404) (width 0.508) (layer B.Cu) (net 33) (status 20))
 (segment (start 41.91 43.2308) (end 47.3196 48.6404) (width 0.508) (layer B.Cu) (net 33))
 (segment (start 44.45 37.592) (end 44.45 44.3484) (width 0.508) (layer B.Cu) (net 34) (status 10))
 (segment (start 46.742 46.6404) (end 100.2792 46.6404) (width 0.508) (layer B.Cu) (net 34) (status 20))
 (segment (start 44.45 44.3484) (end 46.742 46.6404) (width 0.508) (layer B.Cu) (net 34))
 (segment (start 59.69 37.592) (end 61.9252 35.3568) (width 0.508) (layer B.Cu) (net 40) (status 10))
 (segment (start 99.5628 35.3568) (end 100.2792 34.6404) (width 0.508) (layer B.Cu) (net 40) (status 20))
 (segment (start 61.9252 35.3568) (end 99.5628 35.3568) (width 0.508) (layer B.Cu) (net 40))
 (segment (start 99.976799 36.337999) (end 100.2792 36.6404) (width 0.508) (layer B.Cu) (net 39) (status 30))
 (segment (start 63.484001 36.337999) (end 99.976799 36.337999) (width 0.508) (layer B.Cu) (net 39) (status 20))
 (segment (start 62.23 37.592) (end 63.484001 36.337999) (width 0.508) (layer B.Cu) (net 39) (status 10))
 (segment (start 99.604201 39.315399) (end 100.2792 38.6404) (width 0.508) (layer B.Cu) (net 38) (status 20))
 (segment (start 56.333399 39.315399) (end 99.604201 39.315399) (width 0.508) (layer B.Cu) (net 38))
 (segment (start 54.61 37.592) (end 56.333399 39.315399) (width 0.508) (layer B.Cu) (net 38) (status 10))
 (segment (start 55.1184 40.6404) (end 100.2792 40.6404) (width 0.508) (layer B.Cu) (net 37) (status 20))
 (segment (start 52.07 37.592) (end 55.1184 40.6404) (width 0.508) (layer B.Cu) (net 37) (status 10))
 (segment (start 54.5784 42.6404) (end 54.4068 42.4688) (width 0.508) (layer B.Cu) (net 36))
 (segment (start 100.2792 42.6404) (end 54.5784 42.6404) (width 0.508) (layer B.Cu) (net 36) (status 10))
 (segment (start 49.53 37.592) (end 54.4068 42.4688) (width 0.508) (layer B.Cu) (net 36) (status 10))
 (segment (start 46.99 42.672) (end 46.99 37.592) (width 0.508) (layer B.Cu) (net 35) (status 20))
 (segment (start 48.9584 44.6404) (end 46.99 42.672) (width 0.508) (layer B.Cu) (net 35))
 (segment (start 100.2792 44.6404) (end 48.9584 44.6404) (width 0.508) (layer B.Cu) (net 35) (status 10))
 (segment (start 69.1388 73.152) (end 69.1388 62.6222) (width 0.508) (layer F.Cu) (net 5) (status 20))
 (segment (start 74.6272 78.6404) (end 69.1388 73.152) (width 0.508) (layer F.Cu) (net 5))
 (segment (start 100.2792 78.6404) (end 74.6272 78.6404) (width 0.508) (layer F.Cu) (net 5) (status 10))
 (segment (start 76.488 76.6404) (end 100.2792 76.6404) (width 0.508) (layer F.Cu) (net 4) (status 20))
 (segment (start 70.4088 62.6222) (end 70.4088 73.420724) (width 0.508) (layer F.Cu) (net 4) (status 10))
 (segment (start 73.628476 76.6404) (end 76.488 76.6404) (width 0.508) (layer F.Cu) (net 4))
 (segment (start 70.4088 73.420724) (end 73.628476 76.6404) (width 0.508) (layer F.Cu) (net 4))
 (segment (start 27.8384 50.4952) (end 25.9588 50.4952) (width 1.524) (layer PWRGND) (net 1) (status 10))
 (segment (start 100.2792 80.6404) (end 102.0272 80.6404) (width 1.524) (layer PWRGND) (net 1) (status 10))
 (segment (start 100.2792 30.6404) (end 101.846 30.6404) (width 1.524) (layer PWRGND) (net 1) (status 10))
 (segment (start 108.212 30.6404) (end 108.458 30.8864) (width 3.048) (layer PWRGND) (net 1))
 (segment (start 101.846 30.6404) (end 108.212 30.6404) (width 3.048) (layer PWRGND) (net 1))
 (segment (start 108.458 30.8864) (end 108.458 80.772) (width 3.048) (layer PWRGND) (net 1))
 (segment (start 102.0272 80.6404) (end 108.3264 80.6404) (width 3.048) (layer PWRGND) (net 1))
 (segment (start 75.3721 63.7755) (end 76.1492 63.7755) (width 1.016) (layer F.Cu) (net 1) (status 20))
 (segment (start 74.2188 62.6222) (end 75.3721 63.7755) (width 1.016) (layer F.Cu) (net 1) (status 10))
 (via (at 76.1492 63.7755) (size 0.8) (drill 0.4) (layers F.Cu B.Cu) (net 1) (status 30))
 (segment (start 76.1492 63.7755) (end 79.7267 63.7755) (width 1.016) (layer MISC) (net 1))
 (segment (start 79.7267 63.7755) (end 80.264 64.3128) (width 1.016) (layer MISC) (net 1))
 (segment (start 80.264 64.3128) (end 80.264 79.8576) (width 1.016) (layer MISC) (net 1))
 (segment (start 81.0468 80.6404) (end 100.2792 80.6404) (width 1.016) (layer MISC) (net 1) (status 20))
 (segment (start 80.264 79.8576) (end 81.0468 80.6404) (width 1.016) (layer MISC) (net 1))
 (segment (start 25.90139 39.73221) (end 26.4668 39.1668) (width 1.524) (layer PWRGND) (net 1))
 (segment (start 25.90139 50.43779) (end 25.90139 39.73221) (width 1.524) (layer PWRGND) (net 1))
 (segment (start 25.9588 50.4952) (end 25.90139 50.43779) (width 1.524) (layer PWRGND) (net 1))
 (segment (start 76.1492 63.7755) (end 76.1492 63.7755) (width 1.016) (layer F.Cu) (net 1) (status 20))
 (segment (start 33.6804 40.132) (end 36.83 40.132) (width 1.524) (layer PWRGND) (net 1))
 (segment (start 32.7152 39.1668) (end 33.6804 40.132) (width 1.524) (layer PWRGND) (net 1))
 (segment (start 26.4668 39.1668) (end 31.4452 39.1668) (width 1.524) (layer PWRGND) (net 1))
 (segment (start 31.4452 39.1668) (end 32.7152 39.1668) (width 1.524) (layer PWRGND) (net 1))
 (segment (start 31.4452 36.701278) (end 31.4452 39.1668) (width 3.048) (layer PWRGND) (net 1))
 (segment (start 48.994878 19.1516) (end 31.4452 36.701278) (width 3.048) (layer PWRGND) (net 1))
 (segment (start 104.0384 19.1516) (end 48.994878 19.1516) (width 3.048) (layer PWRGND) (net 1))
 (segment (start 108.458 23.5712) (end 104.0384 19.1516) (width 3.048) (layer PWRGND) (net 1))
 (segment (start 108.458 30.8864) (end 108.458 23.5712) (width 3.048) (layer PWRGND) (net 1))
 (segment (start 32.909774 47.1242) (end 33.551974 46.482) (width 0.508) (layer F.Cu) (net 13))
 (segment (start 29.6844 47.1242) (end 32.909774 47.1242) (width 0.508) (layer F.Cu) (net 13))
 (segment (start 33.551974 46.482) (end 35.02 46.482) (width 0.508) (layer F.Cu) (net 13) (status 20))
 (segment (start 28.8134 47.9952) (end 29.6844 47.1242) (width 0.508) (layer F.Cu) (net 13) (status 10))
 (segment (start 27.8384 47.9952) (end 28.8134 47.9952) (width 0.508) (layer F.Cu) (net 13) (status 30))
 (segment (start 33.015986 45.946014) (end 35.02 43.942) (width 0.508) (layer F.Cu) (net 12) (status 20))
 (segment (start 32.5958 46.3662) (end 33.015986 45.946014) (width 0.508) (layer F.Cu) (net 12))
 (segment (start 28.8134 45.4952) (end 29.6844 46.3662) (width 0.508) (layer F.Cu) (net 12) (status 10))
 (segment (start 27.8384 45.4952) (end 28.8134 45.4952) (width 0.508) (layer F.Cu) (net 12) (status 30))
 (segment (start 29.6844 46.3662) (end 32.5958 46.3662) (width 0.508) (layer F.Cu) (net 12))
 (segment (start 49.53 55.668704) (end 78.501696 84.6404) (width 0.508) (layer B.Cu) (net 19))
 (segment (start 78.501696 84.6404) (end 100.2792 84.6404) (width 0.508) (layer B.Cu) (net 19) (status 20))
 (segment (start 49.53 52.832) (end 49.53 55.668704) (width 0.508) (layer B.Cu) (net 19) (status 10))
 (segment (start 46.99 54.12998) (end 79.50042 86.6404) (width 0.508) (layer B.Cu) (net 18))
 (segment (start 79.50042 86.6404) (end 100.2792 86.6404) (width 0.508) (layer B.Cu) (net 18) (status 20))
 (segment (start 46.99 52.832) (end 46.99 54.12998) (width 0.508) (layer B.Cu) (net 18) (status 10))
 (segment (start 80.2584 88.6404) (end 100.2792 88.6404) (width 0.508) (layer B.Cu) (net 17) (status 20))
 (segment (start 44.45 52.832) (end 80.2584 88.6404) (width 0.508) (layer B.Cu) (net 17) (status 10))
 (segment (start 79.7184 90.6404) (end 41.91 52.832) (width 0.508) (layer B.Cu) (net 16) (status 20))
 (segment (start 100.2792 90.6404) (end 79.7184 90.6404) (width 0.508) (layer B.Cu) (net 16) (status 10))
 (segment (start 79.1784 92.6404) (end 100.2792 92.6404) (width 0.508) (layer B.Cu) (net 15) (status 20))
 (segment (start 39.37 52.832) (end 79.1784 92.6404) (width 0.508) (layer B.Cu) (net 15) (status 10))
 (segment (start 78.6384 94.6404) (end 100.2792 94.6404) (width 0.508) (layer B.Cu) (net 14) (status 20))
 (segment (start 36.83 52.832) (end 78.6384 94.6404) (width 0.508) (layer B.Cu) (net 14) (status 10))
 (segment (start 57.15 37.592) (end 61.0108 33.7312) (width 0.508) (layer B.Cu) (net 41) (status 10))
 (segment (start 99.1884 33.7312) (end 100.2792 32.6404) (width 0.508) (layer B.Cu) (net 41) (status 20))
 (segment (start 61.0108 33.7312) (end 99.1884 33.7312) (width 0.508) (layer B.Cu) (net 41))
 (segment (start 71.6788 62.6222) (end 71.6788 64.6684) (width 0.508) (layer F.Cu) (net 3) (status 10))
 (segment (start 71.6788 64.6684) (end 72.9488 65.9384) (width 0.508) (layer F.Cu) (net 3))
 (segment (start 72.9488 65.9384) (end 98.0948 65.9384) (width 0.508) (layer F.Cu) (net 3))
 (segment (start 99.150199 29.769401) (end 100.2792 28.6404) (width 0.508) (layer F.Cu) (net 3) (status 20))
 (segment (start 99.150199 64.883001) (end 99.150199 29.769401) (width 0.508) (layer F.Cu) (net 3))
 (segment (start 98.0948 65.9384) (end 99.150199 64.883001) (width 0.508) (layer F.Cu) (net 3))
 (segment (start 72.9488 64.262) (end 72.9488 62.6222) (width 0.508) (layer F.Cu) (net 2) (status 20))
 (segment (start 73.91719 65.23039) (end 72.9488 64.262) (width 0.508) (layer F.Cu) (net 2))
 (segment (start 97.78681 65.23039) (end 73.91719 65.23039) (width 0.508) (layer F.Cu) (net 2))
 (segment (start 98.250456 64.766744) (end 97.78681 65.23039) (width 0.508) (layer F.Cu) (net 2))
 (segment (start 98.250456 28.669144) (end 98.250456 64.766744) (width 0.508) (layer F.Cu) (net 2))
 (segment (start 100.2792 26.6404) (end 98.250456 28.669144) (width 0.508) (layer F.Cu) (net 2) (status 10))
 (segment (start 76.184001 52.230079) (end 76.184001 57.754099) (width 0.508) (layer F.Cu) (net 6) (status 20))
 (segment (start 75.531921 51.577999) (end 76.184001 52.230079) (width 0.508) (layer F.Cu) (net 6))
 (segment (start 71.104001 51.577999) (end 75.531921 51.577999) (width 0.508) (layer F.Cu) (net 6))
 (segment (start 76.184001 57.754099) (end 76.1492 57.7889) (width 0.508) (layer F.Cu) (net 6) (status 30))
 (segment (start 69.85 52.832) (end 71.104001 51.577999) (width 0.508) (layer F.Cu) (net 6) (status 10))
 (segment (start 74.3355 57.7889) (end 74.2188 57.6722) (width 0.508) (layer F.Cu) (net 6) (status 30))
 (segment (start 76.1492 57.7889) (end 74.3355 57.7889) (width 0.508) (layer F.Cu) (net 6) (status 30))
 (segment (start 73.73161 61.14239) (end 74.2188 60.6552) (width 0.508) (layer F.Cu) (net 6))
 (segment (start 67.10361 61.14239) (end 73.73161 61.14239) (width 0.508) (layer F.Cu) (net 6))
 (segment (start 66.5988 61.6472) (end 67.10361 61.14239) (width 0.508) (layer F.Cu) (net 6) (status 10))
 (segment (start 74.2188 60.6552) (end 74.2188 57.6722) (width 0.508) (layer F.Cu) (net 6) (status 20))
 (segment (start 66.5988 62.6222) (end 66.5988 61.6472) (width 0.508) (layer F.Cu) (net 6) (status 30))
 (segment (start 72.9488 54.8132) (end 74.93 52.832) (width 0.508) (layer F.Cu) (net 11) (status 20))
 (segment (start 72.9488 57.6722) (end 72.9488 54.8132) (width 0.508) (layer F.Cu) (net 11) (status 10))
 (segment (start 71.6788 57.6722) (end 71.6788 56.54359) (width 0.508) (layer F.Cu) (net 10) (status 10))
 (segment (start 72.24079 52.98121) (end 72.39 52.832) (width 0.508) (layer F.Cu) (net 10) (status 30))
 (segment (start 72.24079 55.9816) (end 72.24079 52.98121) (width 0.508) (layer F.Cu) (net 10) (status 20))
 (segment (start 71.6788 56.54359) (end 72.24079 55.9816) (width 0.508) (layer F.Cu) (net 10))
 (segment (start 64.77 52.832) (end 64.77 54.4068) (width 0.508) (layer F.Cu) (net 9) (status 10))
 (segment (start 64.77 54.4068) (end 65.9638 55.6006) (width 0.508) (layer F.Cu) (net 9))
 (via (at 65.9638 55.6006) (size 0.8) (drill 0.4) (layers F.Cu B.Cu) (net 9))
 (via (at 70.4088 57.6722) (size 0.8) (drill 0.4) (layers F.Cu B.Cu) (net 9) (status 30))
 (segment (start 70.4088 56.3372) (end 70.4088 57.6722) (width 0.508) (layer B.Cu) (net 9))
 (segment (start 70.10081 56.02921) (end 70.4088 56.3372) (width 0.508) (layer B.Cu) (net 9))
 (segment (start 66.39241 56.02921) (end 70.10081 56.02921) (width 0.508) (layer B.Cu) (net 9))
 (segment (start 65.9638 55.6006) (end 66.39241 56.02921) (width 0.508) (layer B.Cu) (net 9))
 (segment (start 67.31 50.038) (end 67.31 37.592) (width 0.508) (layer F.Cu) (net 8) (status 20))
 (segment (start 66.055999 53.433921) (end 66.055999 51.292001) (width 0.508) (layer F.Cu) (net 8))
 (segment (start 66.055999 51.292001) (end 67.31 50.038) (width 0.508) (layer F.Cu) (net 8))
 (segment (start 69.1388 57.6722) (end 69.1388 55.6768) (width 0.508) (layer F.Cu) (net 8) (status 10))
 (segment (start 68.034761 54.572761) (end 67.194839 54.572761) (width 0.508) (layer F.Cu) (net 8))
 (segment (start 67.194839 54.572761) (end 66.055999 53.433921) (width 0.508) (layer F.Cu) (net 8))
 (segment (start 69.1388 55.6768) (end 68.034761 54.572761) (width 0.508) (layer F.Cu) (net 8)))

